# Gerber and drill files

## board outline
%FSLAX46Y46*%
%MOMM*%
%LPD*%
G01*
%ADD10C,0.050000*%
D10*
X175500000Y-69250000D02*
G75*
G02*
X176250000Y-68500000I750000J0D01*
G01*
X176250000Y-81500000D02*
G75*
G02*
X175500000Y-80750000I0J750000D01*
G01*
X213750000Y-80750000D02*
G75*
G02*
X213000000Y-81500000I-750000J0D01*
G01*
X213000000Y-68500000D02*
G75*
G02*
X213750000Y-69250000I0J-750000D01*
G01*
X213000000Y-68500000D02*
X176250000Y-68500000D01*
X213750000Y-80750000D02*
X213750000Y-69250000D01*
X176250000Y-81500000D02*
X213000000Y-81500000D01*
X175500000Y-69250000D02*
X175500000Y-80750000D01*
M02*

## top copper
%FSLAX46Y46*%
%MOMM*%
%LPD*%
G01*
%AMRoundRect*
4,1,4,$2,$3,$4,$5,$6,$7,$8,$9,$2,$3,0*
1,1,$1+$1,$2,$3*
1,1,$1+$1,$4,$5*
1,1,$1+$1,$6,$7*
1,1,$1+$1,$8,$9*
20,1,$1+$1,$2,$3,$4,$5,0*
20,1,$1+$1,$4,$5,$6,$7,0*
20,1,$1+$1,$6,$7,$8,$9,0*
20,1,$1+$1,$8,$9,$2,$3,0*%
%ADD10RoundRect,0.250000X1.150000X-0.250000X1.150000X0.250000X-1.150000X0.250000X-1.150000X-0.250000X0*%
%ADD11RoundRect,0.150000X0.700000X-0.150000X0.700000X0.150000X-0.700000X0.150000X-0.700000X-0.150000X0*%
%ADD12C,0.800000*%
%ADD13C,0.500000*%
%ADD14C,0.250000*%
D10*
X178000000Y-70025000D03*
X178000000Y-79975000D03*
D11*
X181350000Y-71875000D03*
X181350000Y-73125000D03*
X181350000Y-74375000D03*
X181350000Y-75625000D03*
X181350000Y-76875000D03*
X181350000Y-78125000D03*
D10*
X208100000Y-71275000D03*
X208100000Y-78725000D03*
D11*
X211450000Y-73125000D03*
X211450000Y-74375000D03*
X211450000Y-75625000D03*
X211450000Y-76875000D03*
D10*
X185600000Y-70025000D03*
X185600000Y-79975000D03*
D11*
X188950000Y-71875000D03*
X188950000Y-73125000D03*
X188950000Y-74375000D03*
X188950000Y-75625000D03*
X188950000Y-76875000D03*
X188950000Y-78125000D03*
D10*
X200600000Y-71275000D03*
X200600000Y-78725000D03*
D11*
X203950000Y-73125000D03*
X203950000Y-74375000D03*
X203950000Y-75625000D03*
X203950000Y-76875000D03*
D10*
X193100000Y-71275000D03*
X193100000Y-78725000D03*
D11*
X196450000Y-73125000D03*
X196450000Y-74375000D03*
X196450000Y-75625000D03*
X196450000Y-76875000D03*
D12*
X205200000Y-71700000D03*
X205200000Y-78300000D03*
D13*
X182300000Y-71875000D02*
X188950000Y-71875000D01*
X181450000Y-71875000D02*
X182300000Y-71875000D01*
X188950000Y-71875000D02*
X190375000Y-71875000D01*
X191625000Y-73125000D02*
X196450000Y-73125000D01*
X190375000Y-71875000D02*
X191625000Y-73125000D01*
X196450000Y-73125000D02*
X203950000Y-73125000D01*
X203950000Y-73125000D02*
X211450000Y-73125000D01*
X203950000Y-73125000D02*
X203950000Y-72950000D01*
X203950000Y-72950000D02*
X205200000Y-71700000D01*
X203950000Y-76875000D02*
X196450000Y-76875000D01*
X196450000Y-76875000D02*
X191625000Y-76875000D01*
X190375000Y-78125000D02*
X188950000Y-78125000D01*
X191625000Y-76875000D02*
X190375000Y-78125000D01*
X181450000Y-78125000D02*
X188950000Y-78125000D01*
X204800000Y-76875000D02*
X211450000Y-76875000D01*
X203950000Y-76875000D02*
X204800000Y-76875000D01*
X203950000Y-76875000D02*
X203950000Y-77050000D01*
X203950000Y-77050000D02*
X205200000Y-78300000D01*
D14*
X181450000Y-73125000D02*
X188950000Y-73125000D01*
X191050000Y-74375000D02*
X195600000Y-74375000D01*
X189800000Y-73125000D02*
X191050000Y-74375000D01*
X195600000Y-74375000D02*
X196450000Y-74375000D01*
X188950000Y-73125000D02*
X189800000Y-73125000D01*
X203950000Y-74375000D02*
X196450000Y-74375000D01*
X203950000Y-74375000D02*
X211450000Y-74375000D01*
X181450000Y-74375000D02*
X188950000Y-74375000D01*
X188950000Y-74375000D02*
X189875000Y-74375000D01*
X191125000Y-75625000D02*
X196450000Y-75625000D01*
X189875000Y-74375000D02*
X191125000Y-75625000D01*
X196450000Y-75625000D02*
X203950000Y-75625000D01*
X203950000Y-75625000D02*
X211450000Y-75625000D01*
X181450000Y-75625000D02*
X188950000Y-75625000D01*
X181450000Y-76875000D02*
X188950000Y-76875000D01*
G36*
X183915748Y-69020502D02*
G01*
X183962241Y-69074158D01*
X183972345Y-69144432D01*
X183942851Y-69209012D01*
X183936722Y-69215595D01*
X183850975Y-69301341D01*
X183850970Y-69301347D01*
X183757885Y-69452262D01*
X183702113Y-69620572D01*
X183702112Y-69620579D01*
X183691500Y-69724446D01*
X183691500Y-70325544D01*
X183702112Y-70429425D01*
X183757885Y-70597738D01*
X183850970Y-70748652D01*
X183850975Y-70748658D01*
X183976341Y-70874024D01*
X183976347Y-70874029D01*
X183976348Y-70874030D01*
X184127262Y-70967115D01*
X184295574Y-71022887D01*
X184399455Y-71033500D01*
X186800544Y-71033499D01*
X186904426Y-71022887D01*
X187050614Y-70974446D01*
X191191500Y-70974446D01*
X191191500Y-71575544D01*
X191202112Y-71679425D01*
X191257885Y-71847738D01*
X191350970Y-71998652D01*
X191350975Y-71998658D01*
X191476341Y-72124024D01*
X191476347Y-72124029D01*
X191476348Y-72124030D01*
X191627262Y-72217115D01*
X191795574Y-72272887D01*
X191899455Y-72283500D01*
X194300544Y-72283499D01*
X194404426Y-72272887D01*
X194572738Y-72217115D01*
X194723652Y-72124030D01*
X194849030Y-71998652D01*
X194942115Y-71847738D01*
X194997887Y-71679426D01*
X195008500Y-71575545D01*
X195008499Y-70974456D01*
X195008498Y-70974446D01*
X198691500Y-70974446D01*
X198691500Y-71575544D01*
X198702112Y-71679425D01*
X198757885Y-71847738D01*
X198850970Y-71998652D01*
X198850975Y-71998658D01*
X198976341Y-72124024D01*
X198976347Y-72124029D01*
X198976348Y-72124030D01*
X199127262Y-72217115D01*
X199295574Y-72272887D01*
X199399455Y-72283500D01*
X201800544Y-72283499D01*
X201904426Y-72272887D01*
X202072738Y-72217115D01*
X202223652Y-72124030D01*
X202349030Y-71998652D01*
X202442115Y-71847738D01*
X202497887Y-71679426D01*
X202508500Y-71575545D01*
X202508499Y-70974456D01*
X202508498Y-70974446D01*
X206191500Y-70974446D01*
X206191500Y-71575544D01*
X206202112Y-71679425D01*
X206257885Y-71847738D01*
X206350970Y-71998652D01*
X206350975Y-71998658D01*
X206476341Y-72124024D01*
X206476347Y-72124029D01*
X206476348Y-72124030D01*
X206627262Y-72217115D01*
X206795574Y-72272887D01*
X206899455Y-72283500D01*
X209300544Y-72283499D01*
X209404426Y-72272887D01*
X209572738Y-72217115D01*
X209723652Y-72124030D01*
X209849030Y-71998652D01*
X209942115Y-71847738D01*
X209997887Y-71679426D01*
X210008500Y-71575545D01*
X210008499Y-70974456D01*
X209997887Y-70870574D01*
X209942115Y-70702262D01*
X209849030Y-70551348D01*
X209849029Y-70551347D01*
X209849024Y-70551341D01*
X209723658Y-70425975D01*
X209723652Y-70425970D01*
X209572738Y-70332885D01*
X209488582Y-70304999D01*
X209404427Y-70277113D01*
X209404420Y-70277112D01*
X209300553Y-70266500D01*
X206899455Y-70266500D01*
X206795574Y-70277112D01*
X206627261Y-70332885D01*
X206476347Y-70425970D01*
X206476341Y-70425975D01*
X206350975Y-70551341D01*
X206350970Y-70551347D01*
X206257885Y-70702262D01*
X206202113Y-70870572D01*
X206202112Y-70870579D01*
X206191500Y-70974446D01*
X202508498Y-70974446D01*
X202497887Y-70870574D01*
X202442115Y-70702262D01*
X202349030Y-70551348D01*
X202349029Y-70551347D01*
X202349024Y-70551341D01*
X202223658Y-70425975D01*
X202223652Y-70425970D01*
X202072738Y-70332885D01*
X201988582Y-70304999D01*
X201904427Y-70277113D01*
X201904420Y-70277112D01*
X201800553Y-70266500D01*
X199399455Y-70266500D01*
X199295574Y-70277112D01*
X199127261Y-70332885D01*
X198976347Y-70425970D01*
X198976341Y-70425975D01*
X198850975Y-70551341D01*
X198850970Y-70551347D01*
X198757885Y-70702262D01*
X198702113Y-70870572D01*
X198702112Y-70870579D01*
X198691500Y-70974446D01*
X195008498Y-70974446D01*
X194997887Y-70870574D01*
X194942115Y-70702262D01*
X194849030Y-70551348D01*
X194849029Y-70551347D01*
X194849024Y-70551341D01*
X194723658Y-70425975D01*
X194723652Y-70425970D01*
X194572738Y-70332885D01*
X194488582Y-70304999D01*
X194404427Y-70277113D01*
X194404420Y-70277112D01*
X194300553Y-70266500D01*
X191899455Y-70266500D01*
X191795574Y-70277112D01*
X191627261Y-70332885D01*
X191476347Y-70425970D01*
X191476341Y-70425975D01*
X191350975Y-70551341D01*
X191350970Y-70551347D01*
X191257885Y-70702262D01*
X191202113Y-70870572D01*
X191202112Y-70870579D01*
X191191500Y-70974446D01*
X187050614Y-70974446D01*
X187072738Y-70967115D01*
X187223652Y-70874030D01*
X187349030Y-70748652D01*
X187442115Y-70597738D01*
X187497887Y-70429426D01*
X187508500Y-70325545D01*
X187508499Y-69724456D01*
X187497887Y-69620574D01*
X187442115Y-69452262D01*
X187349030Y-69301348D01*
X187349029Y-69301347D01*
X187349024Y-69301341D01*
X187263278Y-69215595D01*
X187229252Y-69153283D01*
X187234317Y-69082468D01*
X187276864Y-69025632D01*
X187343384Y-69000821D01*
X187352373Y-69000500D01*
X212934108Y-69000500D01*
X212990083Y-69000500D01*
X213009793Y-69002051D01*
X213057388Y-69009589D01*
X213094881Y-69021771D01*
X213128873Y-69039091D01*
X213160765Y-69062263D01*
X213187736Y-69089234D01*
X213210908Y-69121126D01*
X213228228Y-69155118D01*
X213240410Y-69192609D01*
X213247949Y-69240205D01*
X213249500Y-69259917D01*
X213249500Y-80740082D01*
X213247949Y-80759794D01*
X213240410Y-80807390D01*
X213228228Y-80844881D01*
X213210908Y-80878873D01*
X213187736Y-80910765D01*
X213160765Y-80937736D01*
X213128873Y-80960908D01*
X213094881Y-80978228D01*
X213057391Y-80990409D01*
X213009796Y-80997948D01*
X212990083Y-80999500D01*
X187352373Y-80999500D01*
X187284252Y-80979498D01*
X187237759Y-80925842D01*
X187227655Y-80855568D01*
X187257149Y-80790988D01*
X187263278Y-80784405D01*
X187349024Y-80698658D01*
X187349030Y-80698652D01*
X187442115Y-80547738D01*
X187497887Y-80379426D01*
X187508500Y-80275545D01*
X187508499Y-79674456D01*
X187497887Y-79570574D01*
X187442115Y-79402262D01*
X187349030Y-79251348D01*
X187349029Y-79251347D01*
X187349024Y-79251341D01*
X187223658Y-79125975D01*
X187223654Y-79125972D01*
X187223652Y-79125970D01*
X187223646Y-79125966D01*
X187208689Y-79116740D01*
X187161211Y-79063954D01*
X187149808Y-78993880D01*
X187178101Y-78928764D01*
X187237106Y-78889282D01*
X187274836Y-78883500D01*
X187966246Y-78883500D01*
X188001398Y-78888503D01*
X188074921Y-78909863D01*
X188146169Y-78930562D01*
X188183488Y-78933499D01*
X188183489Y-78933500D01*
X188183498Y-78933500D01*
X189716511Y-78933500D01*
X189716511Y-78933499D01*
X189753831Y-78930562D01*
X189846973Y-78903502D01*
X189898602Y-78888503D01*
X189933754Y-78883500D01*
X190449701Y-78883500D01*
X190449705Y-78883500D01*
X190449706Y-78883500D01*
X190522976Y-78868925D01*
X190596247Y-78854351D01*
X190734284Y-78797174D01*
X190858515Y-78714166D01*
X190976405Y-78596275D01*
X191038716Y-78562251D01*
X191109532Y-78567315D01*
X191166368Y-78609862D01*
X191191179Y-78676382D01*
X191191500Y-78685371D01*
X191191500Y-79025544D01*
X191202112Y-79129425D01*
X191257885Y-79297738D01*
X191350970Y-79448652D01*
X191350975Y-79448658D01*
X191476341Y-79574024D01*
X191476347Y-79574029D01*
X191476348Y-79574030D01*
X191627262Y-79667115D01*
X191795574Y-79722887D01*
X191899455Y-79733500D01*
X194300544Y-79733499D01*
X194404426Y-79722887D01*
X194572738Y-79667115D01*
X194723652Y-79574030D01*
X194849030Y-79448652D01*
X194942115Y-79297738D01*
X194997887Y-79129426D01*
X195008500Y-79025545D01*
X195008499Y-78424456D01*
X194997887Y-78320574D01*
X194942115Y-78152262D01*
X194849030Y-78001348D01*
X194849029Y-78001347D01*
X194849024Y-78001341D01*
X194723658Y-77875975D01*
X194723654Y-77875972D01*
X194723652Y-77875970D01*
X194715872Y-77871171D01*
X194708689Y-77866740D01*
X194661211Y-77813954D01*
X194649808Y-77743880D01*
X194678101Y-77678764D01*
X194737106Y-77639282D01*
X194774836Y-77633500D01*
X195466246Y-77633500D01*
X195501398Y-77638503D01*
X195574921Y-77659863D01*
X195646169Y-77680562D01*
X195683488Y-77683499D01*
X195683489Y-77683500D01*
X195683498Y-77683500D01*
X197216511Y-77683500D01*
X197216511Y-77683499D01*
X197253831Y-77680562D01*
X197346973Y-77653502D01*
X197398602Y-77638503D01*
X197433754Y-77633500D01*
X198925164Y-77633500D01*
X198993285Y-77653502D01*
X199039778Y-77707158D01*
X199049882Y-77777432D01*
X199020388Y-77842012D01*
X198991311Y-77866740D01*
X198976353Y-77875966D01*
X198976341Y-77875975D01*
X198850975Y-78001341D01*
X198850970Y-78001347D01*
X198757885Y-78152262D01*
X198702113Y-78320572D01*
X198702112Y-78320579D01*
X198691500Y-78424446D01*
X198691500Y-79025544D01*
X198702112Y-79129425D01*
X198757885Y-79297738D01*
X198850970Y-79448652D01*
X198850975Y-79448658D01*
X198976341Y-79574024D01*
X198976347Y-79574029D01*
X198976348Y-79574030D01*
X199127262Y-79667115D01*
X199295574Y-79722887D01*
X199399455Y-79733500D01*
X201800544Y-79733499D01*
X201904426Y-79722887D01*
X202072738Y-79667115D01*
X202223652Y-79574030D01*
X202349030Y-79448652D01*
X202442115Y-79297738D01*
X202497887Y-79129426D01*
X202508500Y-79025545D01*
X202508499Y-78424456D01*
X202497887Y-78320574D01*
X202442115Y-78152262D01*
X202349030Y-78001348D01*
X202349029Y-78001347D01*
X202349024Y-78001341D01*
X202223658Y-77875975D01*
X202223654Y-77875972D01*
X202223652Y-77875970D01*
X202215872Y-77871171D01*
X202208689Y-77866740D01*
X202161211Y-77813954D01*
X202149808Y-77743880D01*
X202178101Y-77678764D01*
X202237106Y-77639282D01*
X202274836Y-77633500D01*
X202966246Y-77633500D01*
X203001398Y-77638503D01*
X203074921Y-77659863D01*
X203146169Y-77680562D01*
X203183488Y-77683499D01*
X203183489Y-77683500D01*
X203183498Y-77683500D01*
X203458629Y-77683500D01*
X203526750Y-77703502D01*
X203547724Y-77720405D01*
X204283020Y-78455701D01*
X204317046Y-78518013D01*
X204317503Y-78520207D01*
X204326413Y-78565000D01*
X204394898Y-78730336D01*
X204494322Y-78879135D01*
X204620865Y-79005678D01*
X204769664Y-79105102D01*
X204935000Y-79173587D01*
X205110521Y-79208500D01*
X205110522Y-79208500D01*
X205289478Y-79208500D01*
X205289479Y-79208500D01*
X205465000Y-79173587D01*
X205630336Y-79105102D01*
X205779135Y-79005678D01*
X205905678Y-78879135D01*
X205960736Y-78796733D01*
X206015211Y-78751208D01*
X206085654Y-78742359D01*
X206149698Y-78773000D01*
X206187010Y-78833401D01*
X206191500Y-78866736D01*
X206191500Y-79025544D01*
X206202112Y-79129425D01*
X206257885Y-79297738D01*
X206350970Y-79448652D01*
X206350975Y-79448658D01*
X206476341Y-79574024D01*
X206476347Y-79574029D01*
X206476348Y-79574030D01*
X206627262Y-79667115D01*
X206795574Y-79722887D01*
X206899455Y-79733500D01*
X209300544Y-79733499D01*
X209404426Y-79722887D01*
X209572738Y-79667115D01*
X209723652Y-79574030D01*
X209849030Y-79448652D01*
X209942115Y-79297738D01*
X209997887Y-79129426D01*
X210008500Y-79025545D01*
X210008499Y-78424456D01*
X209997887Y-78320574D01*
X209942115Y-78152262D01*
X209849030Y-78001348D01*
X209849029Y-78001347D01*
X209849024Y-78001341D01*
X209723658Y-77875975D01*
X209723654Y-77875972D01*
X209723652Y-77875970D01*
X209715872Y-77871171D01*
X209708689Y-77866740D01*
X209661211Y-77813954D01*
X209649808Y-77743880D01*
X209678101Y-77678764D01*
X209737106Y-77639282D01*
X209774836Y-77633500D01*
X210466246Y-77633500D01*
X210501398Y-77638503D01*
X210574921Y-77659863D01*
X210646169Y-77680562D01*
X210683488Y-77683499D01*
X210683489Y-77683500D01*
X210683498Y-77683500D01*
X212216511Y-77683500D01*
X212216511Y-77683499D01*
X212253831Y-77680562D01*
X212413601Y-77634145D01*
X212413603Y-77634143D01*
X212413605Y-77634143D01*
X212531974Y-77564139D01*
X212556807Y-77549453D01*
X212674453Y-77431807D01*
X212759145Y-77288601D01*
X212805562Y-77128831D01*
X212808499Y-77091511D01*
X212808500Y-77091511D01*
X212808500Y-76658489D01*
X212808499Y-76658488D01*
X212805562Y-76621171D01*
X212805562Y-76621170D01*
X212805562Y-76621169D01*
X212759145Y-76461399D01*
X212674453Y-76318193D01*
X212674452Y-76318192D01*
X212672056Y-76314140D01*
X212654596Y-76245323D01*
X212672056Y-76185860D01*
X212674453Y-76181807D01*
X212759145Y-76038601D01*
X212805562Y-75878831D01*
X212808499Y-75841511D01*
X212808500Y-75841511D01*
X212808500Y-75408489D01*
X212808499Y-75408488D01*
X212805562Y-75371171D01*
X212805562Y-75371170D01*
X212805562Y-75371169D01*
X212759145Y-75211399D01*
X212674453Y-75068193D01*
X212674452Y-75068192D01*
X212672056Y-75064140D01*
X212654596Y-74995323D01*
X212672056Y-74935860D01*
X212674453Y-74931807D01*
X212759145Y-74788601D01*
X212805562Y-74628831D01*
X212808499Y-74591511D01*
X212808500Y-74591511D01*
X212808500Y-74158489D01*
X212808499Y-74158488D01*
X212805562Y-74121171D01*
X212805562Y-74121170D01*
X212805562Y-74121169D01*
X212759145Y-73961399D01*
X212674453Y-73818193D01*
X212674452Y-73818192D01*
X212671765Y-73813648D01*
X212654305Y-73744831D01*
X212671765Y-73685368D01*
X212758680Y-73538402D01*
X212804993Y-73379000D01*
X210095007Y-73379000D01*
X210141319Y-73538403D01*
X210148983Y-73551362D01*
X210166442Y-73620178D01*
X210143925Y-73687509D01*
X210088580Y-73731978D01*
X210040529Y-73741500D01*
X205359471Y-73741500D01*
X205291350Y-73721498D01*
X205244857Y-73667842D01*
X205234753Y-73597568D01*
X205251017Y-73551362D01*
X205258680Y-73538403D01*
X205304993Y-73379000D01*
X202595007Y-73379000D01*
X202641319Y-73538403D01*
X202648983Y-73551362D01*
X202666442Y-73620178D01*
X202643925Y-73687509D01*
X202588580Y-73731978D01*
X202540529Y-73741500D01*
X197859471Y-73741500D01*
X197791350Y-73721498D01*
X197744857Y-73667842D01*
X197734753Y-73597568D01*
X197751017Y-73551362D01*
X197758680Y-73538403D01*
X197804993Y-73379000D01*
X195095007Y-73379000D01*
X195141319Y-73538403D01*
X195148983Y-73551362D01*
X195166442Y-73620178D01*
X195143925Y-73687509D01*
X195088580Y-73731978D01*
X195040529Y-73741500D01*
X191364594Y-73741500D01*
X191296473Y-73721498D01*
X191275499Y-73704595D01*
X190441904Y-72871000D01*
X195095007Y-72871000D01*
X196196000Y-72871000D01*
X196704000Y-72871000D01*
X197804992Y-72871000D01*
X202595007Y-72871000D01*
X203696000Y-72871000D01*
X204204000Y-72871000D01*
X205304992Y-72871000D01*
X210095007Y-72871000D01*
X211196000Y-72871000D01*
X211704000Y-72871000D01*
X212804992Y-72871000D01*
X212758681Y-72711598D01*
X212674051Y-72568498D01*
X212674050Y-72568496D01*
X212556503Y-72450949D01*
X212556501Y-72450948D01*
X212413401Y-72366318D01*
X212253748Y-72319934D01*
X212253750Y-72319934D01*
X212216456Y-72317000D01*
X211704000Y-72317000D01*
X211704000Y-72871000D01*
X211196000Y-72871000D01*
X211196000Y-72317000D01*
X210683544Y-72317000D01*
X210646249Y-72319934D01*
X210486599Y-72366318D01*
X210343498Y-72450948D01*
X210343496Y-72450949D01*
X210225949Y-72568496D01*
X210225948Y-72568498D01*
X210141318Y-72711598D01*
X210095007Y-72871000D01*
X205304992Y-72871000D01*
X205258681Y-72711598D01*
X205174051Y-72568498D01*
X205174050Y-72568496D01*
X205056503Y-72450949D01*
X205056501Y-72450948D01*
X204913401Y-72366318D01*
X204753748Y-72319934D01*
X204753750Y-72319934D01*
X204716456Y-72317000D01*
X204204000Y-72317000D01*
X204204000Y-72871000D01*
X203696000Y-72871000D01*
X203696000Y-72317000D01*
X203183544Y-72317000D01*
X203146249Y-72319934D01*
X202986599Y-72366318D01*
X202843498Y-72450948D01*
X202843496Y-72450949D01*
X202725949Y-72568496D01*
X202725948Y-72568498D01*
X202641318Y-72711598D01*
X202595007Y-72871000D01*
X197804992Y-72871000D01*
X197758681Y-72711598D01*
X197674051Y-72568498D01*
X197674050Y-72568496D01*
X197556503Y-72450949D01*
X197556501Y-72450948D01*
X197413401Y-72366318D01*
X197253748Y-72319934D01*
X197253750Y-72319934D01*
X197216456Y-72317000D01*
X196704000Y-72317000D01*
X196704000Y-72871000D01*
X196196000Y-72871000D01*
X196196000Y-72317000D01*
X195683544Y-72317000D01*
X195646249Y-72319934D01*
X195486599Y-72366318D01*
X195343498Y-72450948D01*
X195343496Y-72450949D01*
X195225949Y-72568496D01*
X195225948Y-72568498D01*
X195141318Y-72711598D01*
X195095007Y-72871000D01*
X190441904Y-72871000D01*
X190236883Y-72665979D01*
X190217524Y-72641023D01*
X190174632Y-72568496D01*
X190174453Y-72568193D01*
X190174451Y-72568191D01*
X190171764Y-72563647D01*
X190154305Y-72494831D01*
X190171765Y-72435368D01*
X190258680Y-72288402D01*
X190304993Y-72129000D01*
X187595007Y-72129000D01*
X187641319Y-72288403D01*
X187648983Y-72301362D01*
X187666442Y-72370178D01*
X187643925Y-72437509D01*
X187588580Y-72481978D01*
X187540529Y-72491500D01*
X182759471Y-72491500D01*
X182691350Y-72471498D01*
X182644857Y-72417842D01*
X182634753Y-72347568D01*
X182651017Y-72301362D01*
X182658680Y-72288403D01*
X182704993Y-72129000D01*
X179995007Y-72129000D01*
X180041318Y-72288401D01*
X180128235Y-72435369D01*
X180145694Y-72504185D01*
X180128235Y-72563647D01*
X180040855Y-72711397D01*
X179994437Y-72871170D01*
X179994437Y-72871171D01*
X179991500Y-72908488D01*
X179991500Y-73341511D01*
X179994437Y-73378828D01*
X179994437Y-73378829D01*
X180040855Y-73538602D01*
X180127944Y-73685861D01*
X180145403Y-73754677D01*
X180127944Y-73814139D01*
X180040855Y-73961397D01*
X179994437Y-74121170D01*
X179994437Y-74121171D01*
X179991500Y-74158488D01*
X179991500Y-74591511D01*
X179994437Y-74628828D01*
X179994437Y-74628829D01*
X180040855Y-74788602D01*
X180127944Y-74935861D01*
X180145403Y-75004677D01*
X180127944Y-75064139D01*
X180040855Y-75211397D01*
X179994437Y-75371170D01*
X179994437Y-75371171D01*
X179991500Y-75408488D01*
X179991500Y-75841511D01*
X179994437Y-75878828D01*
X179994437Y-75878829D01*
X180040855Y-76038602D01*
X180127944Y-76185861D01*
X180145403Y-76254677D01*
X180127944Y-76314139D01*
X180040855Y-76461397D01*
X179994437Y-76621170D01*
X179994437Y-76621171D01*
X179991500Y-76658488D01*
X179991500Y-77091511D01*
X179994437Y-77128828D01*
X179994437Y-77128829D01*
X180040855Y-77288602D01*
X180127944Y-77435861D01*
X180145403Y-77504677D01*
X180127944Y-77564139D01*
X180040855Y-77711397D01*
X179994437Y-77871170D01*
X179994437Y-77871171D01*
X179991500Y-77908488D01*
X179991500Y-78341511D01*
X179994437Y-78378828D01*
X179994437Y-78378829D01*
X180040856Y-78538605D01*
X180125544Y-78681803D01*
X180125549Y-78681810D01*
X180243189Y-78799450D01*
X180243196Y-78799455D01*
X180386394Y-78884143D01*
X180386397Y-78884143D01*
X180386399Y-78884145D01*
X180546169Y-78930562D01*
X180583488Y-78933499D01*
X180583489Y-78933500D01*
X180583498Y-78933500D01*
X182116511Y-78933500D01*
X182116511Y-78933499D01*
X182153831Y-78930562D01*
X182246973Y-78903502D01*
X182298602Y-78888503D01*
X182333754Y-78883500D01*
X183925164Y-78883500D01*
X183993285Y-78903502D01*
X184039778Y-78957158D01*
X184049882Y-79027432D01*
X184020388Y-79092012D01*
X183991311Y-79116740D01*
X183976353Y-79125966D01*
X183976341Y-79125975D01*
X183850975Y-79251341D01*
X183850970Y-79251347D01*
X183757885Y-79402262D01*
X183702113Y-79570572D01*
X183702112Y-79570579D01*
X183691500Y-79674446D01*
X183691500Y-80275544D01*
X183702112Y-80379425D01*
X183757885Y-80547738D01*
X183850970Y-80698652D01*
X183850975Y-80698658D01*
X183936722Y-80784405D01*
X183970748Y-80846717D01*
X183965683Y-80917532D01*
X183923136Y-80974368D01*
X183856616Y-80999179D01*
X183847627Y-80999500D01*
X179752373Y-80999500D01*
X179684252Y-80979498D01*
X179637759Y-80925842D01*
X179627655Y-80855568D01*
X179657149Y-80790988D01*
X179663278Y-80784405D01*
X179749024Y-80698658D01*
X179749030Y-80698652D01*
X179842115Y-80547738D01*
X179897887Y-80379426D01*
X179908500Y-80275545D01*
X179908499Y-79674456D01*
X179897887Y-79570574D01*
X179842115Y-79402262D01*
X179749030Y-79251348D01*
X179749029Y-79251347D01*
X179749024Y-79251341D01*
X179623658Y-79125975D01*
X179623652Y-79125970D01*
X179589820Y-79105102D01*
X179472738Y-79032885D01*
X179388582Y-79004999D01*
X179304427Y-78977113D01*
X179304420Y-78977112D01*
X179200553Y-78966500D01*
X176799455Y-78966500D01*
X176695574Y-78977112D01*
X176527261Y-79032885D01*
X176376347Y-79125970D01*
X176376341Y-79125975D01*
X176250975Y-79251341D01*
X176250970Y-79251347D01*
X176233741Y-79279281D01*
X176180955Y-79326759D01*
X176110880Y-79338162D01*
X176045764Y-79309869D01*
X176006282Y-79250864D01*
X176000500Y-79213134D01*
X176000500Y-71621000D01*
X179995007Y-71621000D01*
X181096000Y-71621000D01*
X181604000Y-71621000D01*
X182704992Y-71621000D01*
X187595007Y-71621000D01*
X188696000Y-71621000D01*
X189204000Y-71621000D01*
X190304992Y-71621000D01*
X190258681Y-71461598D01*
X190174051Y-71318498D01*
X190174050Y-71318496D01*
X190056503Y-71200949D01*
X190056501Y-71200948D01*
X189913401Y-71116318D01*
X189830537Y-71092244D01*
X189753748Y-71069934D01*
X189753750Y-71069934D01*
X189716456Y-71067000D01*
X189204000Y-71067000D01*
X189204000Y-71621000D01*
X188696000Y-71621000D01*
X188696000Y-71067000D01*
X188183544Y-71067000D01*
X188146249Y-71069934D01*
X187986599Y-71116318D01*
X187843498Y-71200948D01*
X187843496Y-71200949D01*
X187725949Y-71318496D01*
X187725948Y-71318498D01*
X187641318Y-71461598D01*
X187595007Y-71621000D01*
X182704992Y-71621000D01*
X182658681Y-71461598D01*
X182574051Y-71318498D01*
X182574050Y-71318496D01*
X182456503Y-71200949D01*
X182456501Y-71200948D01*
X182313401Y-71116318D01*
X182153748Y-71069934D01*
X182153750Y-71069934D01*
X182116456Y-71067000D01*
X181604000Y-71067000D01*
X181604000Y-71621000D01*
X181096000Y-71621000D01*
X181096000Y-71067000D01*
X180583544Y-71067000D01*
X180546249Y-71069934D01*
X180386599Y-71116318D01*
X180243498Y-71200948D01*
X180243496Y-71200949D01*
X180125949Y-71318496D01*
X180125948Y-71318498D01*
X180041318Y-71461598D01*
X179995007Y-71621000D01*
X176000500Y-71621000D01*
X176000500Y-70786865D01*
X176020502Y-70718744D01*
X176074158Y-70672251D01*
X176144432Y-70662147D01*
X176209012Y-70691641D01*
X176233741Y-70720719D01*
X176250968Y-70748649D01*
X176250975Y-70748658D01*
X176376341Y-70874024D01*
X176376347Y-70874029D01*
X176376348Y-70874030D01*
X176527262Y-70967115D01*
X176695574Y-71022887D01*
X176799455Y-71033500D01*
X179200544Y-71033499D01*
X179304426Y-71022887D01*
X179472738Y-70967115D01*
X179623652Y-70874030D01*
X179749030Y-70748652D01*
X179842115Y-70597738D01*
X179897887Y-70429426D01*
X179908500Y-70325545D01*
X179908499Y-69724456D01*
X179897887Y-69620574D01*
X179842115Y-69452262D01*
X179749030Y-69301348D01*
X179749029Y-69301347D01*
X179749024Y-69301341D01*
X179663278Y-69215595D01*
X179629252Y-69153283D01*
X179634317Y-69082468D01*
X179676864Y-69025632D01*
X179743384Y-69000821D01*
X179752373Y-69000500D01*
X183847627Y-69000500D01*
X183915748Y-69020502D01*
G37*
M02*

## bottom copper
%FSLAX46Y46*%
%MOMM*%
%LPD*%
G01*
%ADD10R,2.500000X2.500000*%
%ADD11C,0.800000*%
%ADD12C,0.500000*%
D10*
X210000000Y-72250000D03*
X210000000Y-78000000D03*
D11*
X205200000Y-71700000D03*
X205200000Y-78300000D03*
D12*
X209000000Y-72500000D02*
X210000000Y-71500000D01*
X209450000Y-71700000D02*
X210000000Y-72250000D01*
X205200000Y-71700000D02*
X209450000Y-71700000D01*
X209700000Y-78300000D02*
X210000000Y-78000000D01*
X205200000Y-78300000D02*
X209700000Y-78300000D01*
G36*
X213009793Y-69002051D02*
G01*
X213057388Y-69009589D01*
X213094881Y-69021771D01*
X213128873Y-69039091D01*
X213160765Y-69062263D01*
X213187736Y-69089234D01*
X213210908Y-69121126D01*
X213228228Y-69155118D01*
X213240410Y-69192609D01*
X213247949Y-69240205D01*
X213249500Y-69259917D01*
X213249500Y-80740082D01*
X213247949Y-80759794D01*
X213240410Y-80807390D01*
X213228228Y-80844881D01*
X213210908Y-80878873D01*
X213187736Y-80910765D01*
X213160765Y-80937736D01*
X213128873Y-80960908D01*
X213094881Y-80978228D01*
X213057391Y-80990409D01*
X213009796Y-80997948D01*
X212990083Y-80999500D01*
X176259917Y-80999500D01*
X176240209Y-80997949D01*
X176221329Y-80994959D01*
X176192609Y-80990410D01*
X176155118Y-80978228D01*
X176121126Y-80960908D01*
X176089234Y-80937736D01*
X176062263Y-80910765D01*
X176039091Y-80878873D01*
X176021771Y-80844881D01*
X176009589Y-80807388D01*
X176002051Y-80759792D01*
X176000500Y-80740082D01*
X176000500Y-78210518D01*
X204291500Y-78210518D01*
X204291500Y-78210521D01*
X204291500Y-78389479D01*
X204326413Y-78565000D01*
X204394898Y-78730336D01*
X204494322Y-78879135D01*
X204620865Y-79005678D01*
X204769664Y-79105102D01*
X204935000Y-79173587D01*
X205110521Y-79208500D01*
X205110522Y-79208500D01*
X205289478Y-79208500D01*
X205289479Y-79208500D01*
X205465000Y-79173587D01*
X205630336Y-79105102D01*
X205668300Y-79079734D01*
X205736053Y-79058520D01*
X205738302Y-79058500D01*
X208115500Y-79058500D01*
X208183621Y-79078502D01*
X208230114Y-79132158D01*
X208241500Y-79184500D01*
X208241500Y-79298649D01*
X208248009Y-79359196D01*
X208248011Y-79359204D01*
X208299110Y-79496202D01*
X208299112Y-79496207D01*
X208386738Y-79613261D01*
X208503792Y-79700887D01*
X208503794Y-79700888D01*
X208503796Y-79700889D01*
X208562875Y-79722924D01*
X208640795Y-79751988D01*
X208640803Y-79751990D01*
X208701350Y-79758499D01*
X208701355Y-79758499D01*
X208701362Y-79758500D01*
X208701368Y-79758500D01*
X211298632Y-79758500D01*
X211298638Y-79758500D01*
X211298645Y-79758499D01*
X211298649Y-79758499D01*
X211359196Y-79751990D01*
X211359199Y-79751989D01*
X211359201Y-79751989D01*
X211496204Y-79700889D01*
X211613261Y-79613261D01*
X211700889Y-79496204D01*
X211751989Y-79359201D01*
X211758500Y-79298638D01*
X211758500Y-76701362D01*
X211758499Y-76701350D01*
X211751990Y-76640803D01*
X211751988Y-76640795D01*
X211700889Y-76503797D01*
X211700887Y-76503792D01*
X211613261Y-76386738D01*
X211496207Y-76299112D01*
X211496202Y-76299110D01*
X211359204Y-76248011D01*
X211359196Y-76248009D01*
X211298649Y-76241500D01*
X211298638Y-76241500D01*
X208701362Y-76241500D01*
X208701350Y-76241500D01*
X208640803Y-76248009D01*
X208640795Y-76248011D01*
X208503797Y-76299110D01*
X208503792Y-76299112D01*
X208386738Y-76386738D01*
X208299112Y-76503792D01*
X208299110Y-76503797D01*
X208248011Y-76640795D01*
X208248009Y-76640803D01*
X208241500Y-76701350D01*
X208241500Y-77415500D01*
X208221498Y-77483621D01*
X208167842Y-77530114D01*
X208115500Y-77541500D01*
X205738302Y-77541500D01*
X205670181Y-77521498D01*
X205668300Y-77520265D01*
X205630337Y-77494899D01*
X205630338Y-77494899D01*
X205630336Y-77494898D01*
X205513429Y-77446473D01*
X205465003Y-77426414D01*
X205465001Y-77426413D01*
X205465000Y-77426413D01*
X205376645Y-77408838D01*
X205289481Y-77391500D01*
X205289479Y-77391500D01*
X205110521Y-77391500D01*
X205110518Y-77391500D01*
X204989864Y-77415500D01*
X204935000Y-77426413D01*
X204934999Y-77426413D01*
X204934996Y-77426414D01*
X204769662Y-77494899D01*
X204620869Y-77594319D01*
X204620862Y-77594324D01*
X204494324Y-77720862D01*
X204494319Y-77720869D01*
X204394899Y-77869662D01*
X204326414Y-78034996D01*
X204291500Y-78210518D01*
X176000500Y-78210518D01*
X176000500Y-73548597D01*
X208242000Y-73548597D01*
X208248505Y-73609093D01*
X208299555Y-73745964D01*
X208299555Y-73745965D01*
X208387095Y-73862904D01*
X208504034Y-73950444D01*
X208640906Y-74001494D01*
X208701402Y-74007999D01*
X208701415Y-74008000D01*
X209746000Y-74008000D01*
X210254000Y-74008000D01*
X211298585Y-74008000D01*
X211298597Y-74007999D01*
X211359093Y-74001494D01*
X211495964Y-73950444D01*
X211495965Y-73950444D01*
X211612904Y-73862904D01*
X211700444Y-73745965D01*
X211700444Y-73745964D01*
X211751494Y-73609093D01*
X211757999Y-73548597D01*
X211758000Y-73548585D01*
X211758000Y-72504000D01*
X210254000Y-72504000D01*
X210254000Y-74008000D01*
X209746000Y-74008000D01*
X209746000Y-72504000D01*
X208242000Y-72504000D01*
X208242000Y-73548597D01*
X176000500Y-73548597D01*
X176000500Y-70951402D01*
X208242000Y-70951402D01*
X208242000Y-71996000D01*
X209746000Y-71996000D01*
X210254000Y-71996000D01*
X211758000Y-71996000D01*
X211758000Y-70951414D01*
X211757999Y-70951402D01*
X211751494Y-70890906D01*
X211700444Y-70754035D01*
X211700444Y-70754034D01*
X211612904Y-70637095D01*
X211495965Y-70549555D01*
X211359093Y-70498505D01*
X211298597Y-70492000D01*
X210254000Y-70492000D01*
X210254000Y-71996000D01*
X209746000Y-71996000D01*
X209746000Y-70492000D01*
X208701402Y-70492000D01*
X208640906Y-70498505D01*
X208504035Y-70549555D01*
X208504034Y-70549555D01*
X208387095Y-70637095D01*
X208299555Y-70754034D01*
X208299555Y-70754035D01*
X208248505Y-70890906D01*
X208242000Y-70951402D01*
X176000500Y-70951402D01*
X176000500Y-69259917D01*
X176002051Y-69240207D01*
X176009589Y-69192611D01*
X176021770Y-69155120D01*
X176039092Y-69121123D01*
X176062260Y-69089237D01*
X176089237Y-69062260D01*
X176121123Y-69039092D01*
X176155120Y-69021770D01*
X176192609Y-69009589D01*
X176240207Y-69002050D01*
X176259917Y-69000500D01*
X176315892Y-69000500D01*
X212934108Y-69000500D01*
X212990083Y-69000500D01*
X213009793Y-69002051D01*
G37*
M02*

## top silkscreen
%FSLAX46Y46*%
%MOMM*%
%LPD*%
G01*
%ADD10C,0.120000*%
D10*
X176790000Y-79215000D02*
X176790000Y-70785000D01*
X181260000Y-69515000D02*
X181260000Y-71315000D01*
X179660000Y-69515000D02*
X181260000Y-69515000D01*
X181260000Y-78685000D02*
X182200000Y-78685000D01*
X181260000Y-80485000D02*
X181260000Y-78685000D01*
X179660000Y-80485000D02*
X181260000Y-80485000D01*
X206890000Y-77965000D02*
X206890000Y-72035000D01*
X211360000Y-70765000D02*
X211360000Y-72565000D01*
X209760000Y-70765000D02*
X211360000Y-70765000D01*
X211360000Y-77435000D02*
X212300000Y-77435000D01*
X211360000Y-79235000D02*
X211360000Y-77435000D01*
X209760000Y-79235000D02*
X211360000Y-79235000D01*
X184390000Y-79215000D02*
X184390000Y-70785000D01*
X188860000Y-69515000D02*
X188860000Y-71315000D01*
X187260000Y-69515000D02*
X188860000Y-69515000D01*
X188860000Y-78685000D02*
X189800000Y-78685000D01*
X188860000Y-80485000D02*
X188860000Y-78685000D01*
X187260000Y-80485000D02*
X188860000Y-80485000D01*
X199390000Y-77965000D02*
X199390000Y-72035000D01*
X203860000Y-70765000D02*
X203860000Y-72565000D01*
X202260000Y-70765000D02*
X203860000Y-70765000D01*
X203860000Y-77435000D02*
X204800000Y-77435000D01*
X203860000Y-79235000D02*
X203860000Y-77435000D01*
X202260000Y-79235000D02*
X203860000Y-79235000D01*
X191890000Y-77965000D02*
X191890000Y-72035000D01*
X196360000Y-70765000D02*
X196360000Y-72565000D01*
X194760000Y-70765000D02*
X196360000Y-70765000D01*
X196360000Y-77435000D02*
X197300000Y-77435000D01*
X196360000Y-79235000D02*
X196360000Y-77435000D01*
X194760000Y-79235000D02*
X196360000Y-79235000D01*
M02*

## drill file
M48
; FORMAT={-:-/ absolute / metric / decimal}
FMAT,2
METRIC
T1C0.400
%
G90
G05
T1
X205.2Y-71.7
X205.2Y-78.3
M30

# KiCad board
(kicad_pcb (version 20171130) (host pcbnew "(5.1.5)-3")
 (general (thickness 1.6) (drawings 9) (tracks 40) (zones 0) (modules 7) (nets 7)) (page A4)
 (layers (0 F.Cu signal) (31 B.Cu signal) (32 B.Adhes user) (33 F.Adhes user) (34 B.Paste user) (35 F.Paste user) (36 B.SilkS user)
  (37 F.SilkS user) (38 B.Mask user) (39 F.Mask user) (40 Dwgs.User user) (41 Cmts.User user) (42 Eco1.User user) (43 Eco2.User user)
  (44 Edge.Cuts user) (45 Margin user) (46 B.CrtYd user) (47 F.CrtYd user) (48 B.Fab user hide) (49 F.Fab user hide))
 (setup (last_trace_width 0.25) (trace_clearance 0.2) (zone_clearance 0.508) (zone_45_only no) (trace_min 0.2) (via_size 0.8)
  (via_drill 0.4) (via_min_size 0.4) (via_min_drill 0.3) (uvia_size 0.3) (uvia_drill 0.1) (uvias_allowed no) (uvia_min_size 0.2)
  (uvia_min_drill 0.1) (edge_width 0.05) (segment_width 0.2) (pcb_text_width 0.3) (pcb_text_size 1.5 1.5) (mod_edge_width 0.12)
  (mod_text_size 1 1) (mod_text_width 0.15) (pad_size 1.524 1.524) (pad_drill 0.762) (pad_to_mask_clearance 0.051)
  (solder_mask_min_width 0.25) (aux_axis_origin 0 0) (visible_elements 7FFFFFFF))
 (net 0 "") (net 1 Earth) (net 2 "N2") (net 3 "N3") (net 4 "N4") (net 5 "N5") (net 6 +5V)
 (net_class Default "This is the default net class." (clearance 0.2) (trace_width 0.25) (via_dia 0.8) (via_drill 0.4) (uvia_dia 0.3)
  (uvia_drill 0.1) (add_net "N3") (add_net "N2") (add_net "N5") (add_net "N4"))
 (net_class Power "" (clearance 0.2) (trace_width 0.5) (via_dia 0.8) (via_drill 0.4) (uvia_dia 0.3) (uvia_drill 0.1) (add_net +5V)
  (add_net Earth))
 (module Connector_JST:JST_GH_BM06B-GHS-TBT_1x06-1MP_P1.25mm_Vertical (layer F.Cu) (at 179.4 75 90)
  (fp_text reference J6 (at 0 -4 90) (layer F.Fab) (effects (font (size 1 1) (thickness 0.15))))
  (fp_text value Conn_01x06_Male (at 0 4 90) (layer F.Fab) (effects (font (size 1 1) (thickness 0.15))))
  (fp_line (start -4.215 -2.61) (end 4.215 -2.61) (layer F.SilkS) (width 0.12))
  (fp_line (start 5.485 1.86) (end 3.685 1.86) (layer F.SilkS) (width 0.12))
  (fp_line (start 5.485 0.26) (end 5.485 1.86) (layer F.SilkS) (width 0.12))
  (fp_line (start -3.685 1.86) (end -3.685 2.8) (layer F.SilkS) (width 0.12))
  (fp_line (start -5.485 1.86) (end -3.685 1.86) (layer F.SilkS) (width 0.12))
  (fp_line (start -5.485 0.26) (end -5.485 1.86) (layer F.SilkS) (width 0.12))
  (pad MP smd roundrect (at 4.975 -1.4 90) (size 1 2.8) (layers F.Cu F.Paste F.Mask) (roundrect_rratio 0.25))
  (pad MP smd roundrect (at -4.975 -1.4 90) (size 1 2.8) (layers F.Cu F.Paste F.Mask) (roundrect_rratio 0.25))
  (pad 6 smd roundrect (at 3.125 1.95 90) (size 0.6 1.7) (layers F.Cu F.Paste F.Mask) (roundrect_rratio 0.25) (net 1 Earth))
  (pad 5 smd roundrect (at 1.875 1.95 90) (size 0.6 1.7) (layers F.Cu F.Paste F.Mask) (roundrect_rratio 0.25) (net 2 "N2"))
  (pad 4 smd roundrect (at 0.625 1.95 90) (size 0.6 1.7) (layers F.Cu F.Paste F.Mask) (roundrect_rratio 0.25) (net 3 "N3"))
  (pad 3 smd roundrect (at -0.625 1.95 90) (size 0.6 1.7) (layers F.Cu F.Paste F.Mask) (roundrect_rratio 0.25) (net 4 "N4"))
  (pad 2 smd roundrect (at -1.875 1.95 90) (size 0.6 1.7) (layers F.Cu F.Paste F.Mask) (roundrect_rratio 0.25) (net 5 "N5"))
  (pad 1 smd roundrect (at -3.125 1.95 90) (size 0.6 1.7) (layers F.Cu F.Paste F.Mask) (roundrect_rratio 0.25) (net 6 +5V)))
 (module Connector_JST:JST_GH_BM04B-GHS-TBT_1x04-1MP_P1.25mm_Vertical (layer F.Cu) (at 209.5 75 90)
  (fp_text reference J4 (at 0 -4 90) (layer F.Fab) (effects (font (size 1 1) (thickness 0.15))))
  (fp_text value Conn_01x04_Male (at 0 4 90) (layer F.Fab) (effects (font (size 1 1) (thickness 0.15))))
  (fp_line (start -2.965 -2.61) (end 2.965 -2.61) (layer F.SilkS) (width 0.12))
  (fp_line (start 4.235 1.86) (end 2.435 1.86) (layer F.SilkS) (width 0.12))
  (fp_line (start 4.235 0.26) (end 4.235 1.86) (layer F.SilkS) (width 0.12))
  (fp_line (start -2.435 1.86) (end -2.435 2.8) (layer F.SilkS) (width 0.12))
  (fp_line (start -4.235 1.86) (end -2.435 1.86) (layer F.SilkS) (width 0.12))
  (fp_line (start -4.235 0.26) (end -4.235 1.86) (layer F.SilkS) (width 0.12))
  (pad MP smd roundrect (at 3.725 -1.4 90) (size 1 2.8) (layers F.Cu F.Paste F.Mask) (roundrect_rratio 0.25))
  (pad MP smd roundrect (at -3.725 -1.4 90) (size 1 2.8) (layers F.Cu F.Paste F.Mask) (roundrect_rratio 0.25))
  (pad 4 smd roundrect (at 1.875 1.95 90) (size 0.6 1.7) (layers F.Cu F.Paste F.Mask) (roundrect_rratio 0.25) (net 1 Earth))
  (pad 3 smd roundrect (at 0.625 1.95 90) (size 0.6 1.7) (layers F.Cu F.Paste F.Mask) (roundrect_rratio 0.25) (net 2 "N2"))
  (pad 2 smd roundrect (at -0.625 1.95 90) (size 0.6 1.7) (layers F.Cu F.Paste F.Mask) (roundrect_rratio 0.25) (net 3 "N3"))
  (pad 1 smd roundrect (at -1.875 1.95 90) (size 0.6 1.7) (layers F.Cu F.Paste F.Mask) (roundrect_rratio 0.25) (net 6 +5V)))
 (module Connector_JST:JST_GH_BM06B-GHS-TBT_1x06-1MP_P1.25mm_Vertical (layer F.Cu) (at 187 75 90)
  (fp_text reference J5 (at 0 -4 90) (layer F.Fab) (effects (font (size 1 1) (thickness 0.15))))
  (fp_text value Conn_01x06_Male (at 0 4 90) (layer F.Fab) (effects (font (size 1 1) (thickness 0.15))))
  (fp_line (start -4.215 -2.61) (end 4.215 -2.61) (layer F.SilkS) (width 0.12))
  (fp_line (start 5.485 1.86) (end 3.685 1.86) (layer F.SilkS) (width 0.12))
  (fp_line (start 5.485 0.26) (end 5.485 1.86) (layer F.SilkS) (width 0.12))
  (fp_line (start -3.685 1.86) (end -3.685 2.8) (layer F.SilkS) (width 0.12))
  (fp_line (start -5.485 1.86) (end -3.685 1.86) (layer F.SilkS) (width 0.12))
  (fp_line (start -5.485 0.26) (end -5.485 1.86) (layer F.SilkS) (width 0.12))
  (pad MP smd roundrect (at 4.975 -1.4 90) (size 1 2.8) (layers F.Cu F.Paste F.Mask) (roundrect_rratio 0.25))
  (pad MP smd roundrect (at -4.975 -1.4 90) (size 1 2.8) (layers F.Cu F.Paste F.Mask) (roundrect_rratio 0.25))
  (pad 6 smd roundrect (at 3.125 1.95 90) (size 0.6 1.7) (layers F.Cu F.Paste F.Mask) (roundrect_rratio 0.25) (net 1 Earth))
  (pad 5 smd roundrect (at 1.875 1.95 90) (size 0.6 1.7) (layers F.Cu F.Paste F.Mask) (roundrect_rratio 0.25) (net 2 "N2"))
  (pad 4 smd roundrect (at 0.625 1.95 90) (size 0.6 1.7) (layers F.Cu F.Paste F.Mask) (roundrect_rratio 0.25) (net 3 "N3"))
  (pad 3 smd roundrect (at -0.625 1.95 90) (size 0.6 1.7) (layers F.Cu F.Paste F.Mask) (roundrect_rratio 0.25) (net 4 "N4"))
  (pad 2 smd roundrect (at -1.875 1.95 90) (size 0.6 1.7) (layers F.Cu F.Paste F.Mask) (roundrect_rratio 0.25) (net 5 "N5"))
  (pad 1 smd roundrect (at -3.125 1.95 90) (size 0.6 1.7) (layers F.Cu F.Paste F.Mask) (roundrect_rratio 0.25) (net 6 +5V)))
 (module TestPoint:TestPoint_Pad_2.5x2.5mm (layer B.Cu) (at 210 72.25)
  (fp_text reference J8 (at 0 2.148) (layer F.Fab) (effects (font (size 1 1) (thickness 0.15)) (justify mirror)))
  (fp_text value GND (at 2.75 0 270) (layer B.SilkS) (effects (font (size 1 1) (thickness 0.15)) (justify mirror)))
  (pad 1 smd rect (at 0 0) (size 2.5 2.5) (layers B.Cu B.Mask) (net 1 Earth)))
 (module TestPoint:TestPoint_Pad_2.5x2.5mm (layer B.Cu) (at 210 78)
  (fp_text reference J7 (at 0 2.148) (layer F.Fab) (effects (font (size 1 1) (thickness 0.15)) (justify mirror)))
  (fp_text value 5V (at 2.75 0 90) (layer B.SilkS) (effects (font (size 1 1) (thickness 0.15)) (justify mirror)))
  (pad 1 smd rect (at 0 0) (size 2.5 2.5) (layers B.Cu B.Mask) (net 6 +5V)))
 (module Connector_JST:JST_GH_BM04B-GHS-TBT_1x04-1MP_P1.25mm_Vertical (layer F.Cu) (at 202 75 90)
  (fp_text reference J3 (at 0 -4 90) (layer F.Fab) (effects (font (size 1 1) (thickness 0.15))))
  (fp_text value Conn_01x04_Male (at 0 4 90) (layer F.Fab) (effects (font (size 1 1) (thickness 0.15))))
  (fp_line (start -2.965 -2.61) (end 2.965 -2.61) (layer F.SilkS) (width 0.12))
  (fp_line (start 4.235 1.86) (end 2.435 1.86) (layer F.SilkS) (width 0.12))
  (fp_line (start 4.235 0.26) (end 4.235 1.86) (layer F.SilkS) (width 0.12))
  (fp_line (start -2.435 1.86) (end -2.435 2.8) (layer F.SilkS) (width 0.12))
  (fp_line (start -4.235 1.86) (end -2.435 1.86) (layer F.SilkS) (width 0.12))
  (fp_line (start -4.235 0.26) (end -4.235 1.86) (layer F.SilkS) (width 0.12))
  (pad MP smd roundrect (at 3.725 -1.4 90) (size 1 2.8) (layers F.Cu F.Paste F.Mask) (roundrect_rratio 0.25))
  (pad MP smd roundrect (at -3.725 -1.4 90) (size 1 2.8) (layers F.Cu F.Paste F.Mask) (roundrect_rratio 0.25))
  (pad 4 smd roundrect (at 1.875 1.95 90) (size 0.6 1.7) (layers F.Cu F.Paste F.Mask) (roundrect_rratio 0.25) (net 1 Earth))
  (pad 3 smd roundrect (at 0.625 1.95 90) (size 0.6 1.7) (layers F.Cu F.Paste F.Mask) (roundrect_rratio 0.25) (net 2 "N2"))
  (pad 2 smd roundrect (at -0.625 1.95 90) (size 0.6 1.7) (layers F.Cu F.Paste F.Mask) (roundrect_rratio 0.25) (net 3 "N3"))
  (pad 1 smd roundrect (at -1.875 1.95 90) (size 0.6 1.7) (layers F.Cu F.Paste F.Mask) (roundrect_rratio 0.25) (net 6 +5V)))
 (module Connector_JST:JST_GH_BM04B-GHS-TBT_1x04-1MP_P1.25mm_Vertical (layer F.Cu) (at 194.5 75 90)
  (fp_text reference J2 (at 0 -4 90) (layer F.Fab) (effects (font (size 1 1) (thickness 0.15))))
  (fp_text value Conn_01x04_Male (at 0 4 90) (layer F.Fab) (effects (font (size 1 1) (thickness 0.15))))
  (fp_line (start -2.965 -2.61) (end 2.965 -2.61) (layer F.SilkS) (width 0.12))
  (fp_line (start 4.235 1.86) (end 2.435 1.86) (layer F.SilkS) (width 0.12))
  (fp_line (start 4.235 0.26) (end 4.235 1.86) (layer F.SilkS) (width 0.12))
  (fp_line (start -2.435 1.86) (end -2.435 2.8) (layer F.SilkS) (width 0.12))
  (fp_line (start -4.235 1.86) (end -2.435 1.86) (layer F.SilkS) (width 0.12))
  (fp_line (start -4.235 0.26) (end -4.235 1.86) (layer F.SilkS) (width 0.12))
  (pad MP smd roundrect (at 3.725 -1.4 90) (size 1 2.8) (layers F.Cu F.Paste F.Mask) (roundrect_rratio 0.25))
  (pad MP smd roundrect (at -3.725 -1.4 90) (size 1 2.8) (layers F.Cu F.Paste F.Mask) (roundrect_rratio 0.25))
  (pad 4 smd roundrect (at 1.875 1.95 90) (size 0.6 1.7) (layers F.Cu F.Paste F.Mask) (roundrect_rratio 0.25) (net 1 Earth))
  (pad 3 smd roundrect (at 0.625 1.95 90) (size 0.6 1.7) (layers F.Cu F.Paste F.Mask) (roundrect_rratio 0.25) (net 2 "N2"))
  (pad 2 smd roundrect (at -0.625 1.95 90) (size 0.6 1.7) (layers F.Cu F.Paste F.Mask) (roundrect_rratio 0.25) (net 3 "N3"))
  (pad 1 smd roundrect (at -1.875 1.95 90) (size 0.6 1.7) (layers F.Cu F.Paste F.Mask) (roundrect_rratio 0.25) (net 6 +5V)))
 (gr_arc (start 176.25 69.25) (end 176.25 68.5) (angle -90) (layer Edge.Cuts) (width 0.05))
 (gr_arc (start 176.25 80.75) (end 175.5 80.75) (angle -90) (layer Edge.Cuts) (width 0.05))
 (gr_arc (start 213 80.75) (end 213 81.5) (angle -90) (layer Edge.Cuts) (width 0.05))
 (gr_arc (start 213 69.25) (end 213.75 69.25) (angle -90) (layer Edge.Cuts) (width 0.05))
 (gr_line (start 213 68.5) (end 176.25 68.5) (layer Edge.Cuts) (width 0.05))
 (gr_line (start 213.75 80.75) (end 213.75 69.25) (layer Edge.Cuts) (width 0.05))
 (gr_line (start 176.25 81.5) (end 213 81.5) (layer Edge.Cuts) (width 0.05))
 (gr_line (start 175.5 69.25) (end 175.5 80.75) (layer Edge.Cuts) (width 0.05))
 (segment (start 209 72.5) (end 210 71.5) (width 0.5) (layer B.Cu) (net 1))
 (segment (start 182.3 71.875) (end 188.95 71.875) (width 0.5) (layer F.Cu) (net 1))
 (segment (start 181.45 71.875) (end 182.3 71.875) (width 0.5) (layer F.Cu) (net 1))
 (segment (start 188.95 71.875) (end 190.375 71.875) (width 0.5) (layer F.Cu) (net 1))
 (segment (start 191.625 73.125) (end 196.45 73.125) (width 0.5) (layer F.Cu) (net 1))
 (segment (start 190.375 71.875) (end 191.625 73.125) (width 0.5) (layer F.Cu) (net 1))
 (segment (start 196.45 73.125) (end 203.95 73.125) (width 0.5) (layer F.Cu) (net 1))
 (segment (start 203.95 73.125) (end 211.45 73.125) (width 0.5) (layer F.Cu) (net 1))
 (via (at 205.2 71.7) (size 0.8) (drill 0.4) (layers F.Cu B.Cu) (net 1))
 (segment (start 203.95 73.125) (end 203.95 72.95) (width 0.5) (layer F.Cu) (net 1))
 (segment (start 203.95 72.95) (end 205.2 71.7) (width 0.5) (layer F.Cu) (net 1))
 (segment (start 209.45 71.7) (end 210 72.25) (width 0.5) (layer B.Cu) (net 1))
 (segment (start 205.2 71.7) (end 209.45 71.7) (width 0.5) (layer B.Cu) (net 1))
 (segment (start 203.95 76.875) (end 196.45 76.875) (width 0.5) (layer F.Cu) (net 6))
 (segment (start 196.45 76.875) (end 191.625 76.875) (width 0.5) (layer F.Cu) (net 6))
 (segment (start 190.375 78.125) (end 188.95 78.125) (width 0.5) (layer F.Cu) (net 6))
 (segment (start 191.625 76.875) (end 190.375 78.125) (width 0.5) (layer F.Cu) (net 6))
 (segment (start 181.45 78.125) (end 188.95 78.125) (width 0.5) (layer F.Cu) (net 6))
 (segment (start 204.8 76.875) (end 211.45 76.875) (width 0.5) (layer F.Cu) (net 6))
 (segment (start 203.95 76.875) (end 204.8 76.875) (width 0.5) (layer F.Cu) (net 6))
 (via (at 205.2 78.3) (size 0.8) (drill 0.4) (layers F.Cu B.Cu) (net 6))
 (segment (start 203.95 76.875) (end 203.95 77.05) (width 0.5) (layer F.Cu) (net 6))
 (segment (start 203.95 77.05) (end 205.2 78.3) (width 0.5) (layer F.Cu) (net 6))
 (segment (start 209.7 78.3) (end 210 78) (width 0.5) (layer B.Cu) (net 6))
 (segment (start 205.2 78.3) (end 209.7 78.3) (width 0.5) (layer B.Cu) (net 6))
 (segment (start 181.45 73.125) (end 188.95 73.125) (width 0.25) (layer F.Cu) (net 2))
 (segment (start 191.05 74.375) (end 195.6 74.375) (width 0.25) (layer F.Cu) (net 2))
 (segment (start 189.8 73.125) (end 191.05 74.375) (width 0.25) (layer F.Cu) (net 2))
 (segment (start 195.6 74.375) (end 196.45 74.375) (width 0.25) (layer F.Cu) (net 2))
 (segment (start 188.95 73.125) (end 189.8 73.125) (width 0.25) (layer F.Cu) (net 2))
 (segment (start 203.95 74.375) (end 196.45 74.375) (width 0.25) (layer F.Cu) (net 2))
 (segment (start 203.95 74.375) (end 211.45 74.375) (width 0.25) (layer F.Cu) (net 2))
 (segment (start 181.45 74.375) (end 188.95 74.375) (width 0.25) (layer F.Cu) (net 3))
 (segment (start 188.95 74.375) (end 189.875 74.375) (width 0.25) (layer F.Cu) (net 3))
 (segment (start 191.125 75.625) (end 196.45 75.625) (width 0.25) (layer F.Cu) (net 3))
 (segment (start 189.875 74.375) (end 191.125 75.625) (width 0.25) (layer F.Cu) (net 3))
 (segment (start 196.45 75.625) (end 203.95 75.625) (width 0.25) (layer F.Cu) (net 3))
 (segment (start 203.95 75.625) (end 211.45 75.625) (width 0.25) (layer F.Cu) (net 3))
 (segment (start 181.45 75.625) (end 188.95 75.625) (width 0.25) (layer F.Cu) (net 4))
 (segment (start 181.45 76.875) (end 188.95 76.875) (width 0.25) (layer F.Cu) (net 5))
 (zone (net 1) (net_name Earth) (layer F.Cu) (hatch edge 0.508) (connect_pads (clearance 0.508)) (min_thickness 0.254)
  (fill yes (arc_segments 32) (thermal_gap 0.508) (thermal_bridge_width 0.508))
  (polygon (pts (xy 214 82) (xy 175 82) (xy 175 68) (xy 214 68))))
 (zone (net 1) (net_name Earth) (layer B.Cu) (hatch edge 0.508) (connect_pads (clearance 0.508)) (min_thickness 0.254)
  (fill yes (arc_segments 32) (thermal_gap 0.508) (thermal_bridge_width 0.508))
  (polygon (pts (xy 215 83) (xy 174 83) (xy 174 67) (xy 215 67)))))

